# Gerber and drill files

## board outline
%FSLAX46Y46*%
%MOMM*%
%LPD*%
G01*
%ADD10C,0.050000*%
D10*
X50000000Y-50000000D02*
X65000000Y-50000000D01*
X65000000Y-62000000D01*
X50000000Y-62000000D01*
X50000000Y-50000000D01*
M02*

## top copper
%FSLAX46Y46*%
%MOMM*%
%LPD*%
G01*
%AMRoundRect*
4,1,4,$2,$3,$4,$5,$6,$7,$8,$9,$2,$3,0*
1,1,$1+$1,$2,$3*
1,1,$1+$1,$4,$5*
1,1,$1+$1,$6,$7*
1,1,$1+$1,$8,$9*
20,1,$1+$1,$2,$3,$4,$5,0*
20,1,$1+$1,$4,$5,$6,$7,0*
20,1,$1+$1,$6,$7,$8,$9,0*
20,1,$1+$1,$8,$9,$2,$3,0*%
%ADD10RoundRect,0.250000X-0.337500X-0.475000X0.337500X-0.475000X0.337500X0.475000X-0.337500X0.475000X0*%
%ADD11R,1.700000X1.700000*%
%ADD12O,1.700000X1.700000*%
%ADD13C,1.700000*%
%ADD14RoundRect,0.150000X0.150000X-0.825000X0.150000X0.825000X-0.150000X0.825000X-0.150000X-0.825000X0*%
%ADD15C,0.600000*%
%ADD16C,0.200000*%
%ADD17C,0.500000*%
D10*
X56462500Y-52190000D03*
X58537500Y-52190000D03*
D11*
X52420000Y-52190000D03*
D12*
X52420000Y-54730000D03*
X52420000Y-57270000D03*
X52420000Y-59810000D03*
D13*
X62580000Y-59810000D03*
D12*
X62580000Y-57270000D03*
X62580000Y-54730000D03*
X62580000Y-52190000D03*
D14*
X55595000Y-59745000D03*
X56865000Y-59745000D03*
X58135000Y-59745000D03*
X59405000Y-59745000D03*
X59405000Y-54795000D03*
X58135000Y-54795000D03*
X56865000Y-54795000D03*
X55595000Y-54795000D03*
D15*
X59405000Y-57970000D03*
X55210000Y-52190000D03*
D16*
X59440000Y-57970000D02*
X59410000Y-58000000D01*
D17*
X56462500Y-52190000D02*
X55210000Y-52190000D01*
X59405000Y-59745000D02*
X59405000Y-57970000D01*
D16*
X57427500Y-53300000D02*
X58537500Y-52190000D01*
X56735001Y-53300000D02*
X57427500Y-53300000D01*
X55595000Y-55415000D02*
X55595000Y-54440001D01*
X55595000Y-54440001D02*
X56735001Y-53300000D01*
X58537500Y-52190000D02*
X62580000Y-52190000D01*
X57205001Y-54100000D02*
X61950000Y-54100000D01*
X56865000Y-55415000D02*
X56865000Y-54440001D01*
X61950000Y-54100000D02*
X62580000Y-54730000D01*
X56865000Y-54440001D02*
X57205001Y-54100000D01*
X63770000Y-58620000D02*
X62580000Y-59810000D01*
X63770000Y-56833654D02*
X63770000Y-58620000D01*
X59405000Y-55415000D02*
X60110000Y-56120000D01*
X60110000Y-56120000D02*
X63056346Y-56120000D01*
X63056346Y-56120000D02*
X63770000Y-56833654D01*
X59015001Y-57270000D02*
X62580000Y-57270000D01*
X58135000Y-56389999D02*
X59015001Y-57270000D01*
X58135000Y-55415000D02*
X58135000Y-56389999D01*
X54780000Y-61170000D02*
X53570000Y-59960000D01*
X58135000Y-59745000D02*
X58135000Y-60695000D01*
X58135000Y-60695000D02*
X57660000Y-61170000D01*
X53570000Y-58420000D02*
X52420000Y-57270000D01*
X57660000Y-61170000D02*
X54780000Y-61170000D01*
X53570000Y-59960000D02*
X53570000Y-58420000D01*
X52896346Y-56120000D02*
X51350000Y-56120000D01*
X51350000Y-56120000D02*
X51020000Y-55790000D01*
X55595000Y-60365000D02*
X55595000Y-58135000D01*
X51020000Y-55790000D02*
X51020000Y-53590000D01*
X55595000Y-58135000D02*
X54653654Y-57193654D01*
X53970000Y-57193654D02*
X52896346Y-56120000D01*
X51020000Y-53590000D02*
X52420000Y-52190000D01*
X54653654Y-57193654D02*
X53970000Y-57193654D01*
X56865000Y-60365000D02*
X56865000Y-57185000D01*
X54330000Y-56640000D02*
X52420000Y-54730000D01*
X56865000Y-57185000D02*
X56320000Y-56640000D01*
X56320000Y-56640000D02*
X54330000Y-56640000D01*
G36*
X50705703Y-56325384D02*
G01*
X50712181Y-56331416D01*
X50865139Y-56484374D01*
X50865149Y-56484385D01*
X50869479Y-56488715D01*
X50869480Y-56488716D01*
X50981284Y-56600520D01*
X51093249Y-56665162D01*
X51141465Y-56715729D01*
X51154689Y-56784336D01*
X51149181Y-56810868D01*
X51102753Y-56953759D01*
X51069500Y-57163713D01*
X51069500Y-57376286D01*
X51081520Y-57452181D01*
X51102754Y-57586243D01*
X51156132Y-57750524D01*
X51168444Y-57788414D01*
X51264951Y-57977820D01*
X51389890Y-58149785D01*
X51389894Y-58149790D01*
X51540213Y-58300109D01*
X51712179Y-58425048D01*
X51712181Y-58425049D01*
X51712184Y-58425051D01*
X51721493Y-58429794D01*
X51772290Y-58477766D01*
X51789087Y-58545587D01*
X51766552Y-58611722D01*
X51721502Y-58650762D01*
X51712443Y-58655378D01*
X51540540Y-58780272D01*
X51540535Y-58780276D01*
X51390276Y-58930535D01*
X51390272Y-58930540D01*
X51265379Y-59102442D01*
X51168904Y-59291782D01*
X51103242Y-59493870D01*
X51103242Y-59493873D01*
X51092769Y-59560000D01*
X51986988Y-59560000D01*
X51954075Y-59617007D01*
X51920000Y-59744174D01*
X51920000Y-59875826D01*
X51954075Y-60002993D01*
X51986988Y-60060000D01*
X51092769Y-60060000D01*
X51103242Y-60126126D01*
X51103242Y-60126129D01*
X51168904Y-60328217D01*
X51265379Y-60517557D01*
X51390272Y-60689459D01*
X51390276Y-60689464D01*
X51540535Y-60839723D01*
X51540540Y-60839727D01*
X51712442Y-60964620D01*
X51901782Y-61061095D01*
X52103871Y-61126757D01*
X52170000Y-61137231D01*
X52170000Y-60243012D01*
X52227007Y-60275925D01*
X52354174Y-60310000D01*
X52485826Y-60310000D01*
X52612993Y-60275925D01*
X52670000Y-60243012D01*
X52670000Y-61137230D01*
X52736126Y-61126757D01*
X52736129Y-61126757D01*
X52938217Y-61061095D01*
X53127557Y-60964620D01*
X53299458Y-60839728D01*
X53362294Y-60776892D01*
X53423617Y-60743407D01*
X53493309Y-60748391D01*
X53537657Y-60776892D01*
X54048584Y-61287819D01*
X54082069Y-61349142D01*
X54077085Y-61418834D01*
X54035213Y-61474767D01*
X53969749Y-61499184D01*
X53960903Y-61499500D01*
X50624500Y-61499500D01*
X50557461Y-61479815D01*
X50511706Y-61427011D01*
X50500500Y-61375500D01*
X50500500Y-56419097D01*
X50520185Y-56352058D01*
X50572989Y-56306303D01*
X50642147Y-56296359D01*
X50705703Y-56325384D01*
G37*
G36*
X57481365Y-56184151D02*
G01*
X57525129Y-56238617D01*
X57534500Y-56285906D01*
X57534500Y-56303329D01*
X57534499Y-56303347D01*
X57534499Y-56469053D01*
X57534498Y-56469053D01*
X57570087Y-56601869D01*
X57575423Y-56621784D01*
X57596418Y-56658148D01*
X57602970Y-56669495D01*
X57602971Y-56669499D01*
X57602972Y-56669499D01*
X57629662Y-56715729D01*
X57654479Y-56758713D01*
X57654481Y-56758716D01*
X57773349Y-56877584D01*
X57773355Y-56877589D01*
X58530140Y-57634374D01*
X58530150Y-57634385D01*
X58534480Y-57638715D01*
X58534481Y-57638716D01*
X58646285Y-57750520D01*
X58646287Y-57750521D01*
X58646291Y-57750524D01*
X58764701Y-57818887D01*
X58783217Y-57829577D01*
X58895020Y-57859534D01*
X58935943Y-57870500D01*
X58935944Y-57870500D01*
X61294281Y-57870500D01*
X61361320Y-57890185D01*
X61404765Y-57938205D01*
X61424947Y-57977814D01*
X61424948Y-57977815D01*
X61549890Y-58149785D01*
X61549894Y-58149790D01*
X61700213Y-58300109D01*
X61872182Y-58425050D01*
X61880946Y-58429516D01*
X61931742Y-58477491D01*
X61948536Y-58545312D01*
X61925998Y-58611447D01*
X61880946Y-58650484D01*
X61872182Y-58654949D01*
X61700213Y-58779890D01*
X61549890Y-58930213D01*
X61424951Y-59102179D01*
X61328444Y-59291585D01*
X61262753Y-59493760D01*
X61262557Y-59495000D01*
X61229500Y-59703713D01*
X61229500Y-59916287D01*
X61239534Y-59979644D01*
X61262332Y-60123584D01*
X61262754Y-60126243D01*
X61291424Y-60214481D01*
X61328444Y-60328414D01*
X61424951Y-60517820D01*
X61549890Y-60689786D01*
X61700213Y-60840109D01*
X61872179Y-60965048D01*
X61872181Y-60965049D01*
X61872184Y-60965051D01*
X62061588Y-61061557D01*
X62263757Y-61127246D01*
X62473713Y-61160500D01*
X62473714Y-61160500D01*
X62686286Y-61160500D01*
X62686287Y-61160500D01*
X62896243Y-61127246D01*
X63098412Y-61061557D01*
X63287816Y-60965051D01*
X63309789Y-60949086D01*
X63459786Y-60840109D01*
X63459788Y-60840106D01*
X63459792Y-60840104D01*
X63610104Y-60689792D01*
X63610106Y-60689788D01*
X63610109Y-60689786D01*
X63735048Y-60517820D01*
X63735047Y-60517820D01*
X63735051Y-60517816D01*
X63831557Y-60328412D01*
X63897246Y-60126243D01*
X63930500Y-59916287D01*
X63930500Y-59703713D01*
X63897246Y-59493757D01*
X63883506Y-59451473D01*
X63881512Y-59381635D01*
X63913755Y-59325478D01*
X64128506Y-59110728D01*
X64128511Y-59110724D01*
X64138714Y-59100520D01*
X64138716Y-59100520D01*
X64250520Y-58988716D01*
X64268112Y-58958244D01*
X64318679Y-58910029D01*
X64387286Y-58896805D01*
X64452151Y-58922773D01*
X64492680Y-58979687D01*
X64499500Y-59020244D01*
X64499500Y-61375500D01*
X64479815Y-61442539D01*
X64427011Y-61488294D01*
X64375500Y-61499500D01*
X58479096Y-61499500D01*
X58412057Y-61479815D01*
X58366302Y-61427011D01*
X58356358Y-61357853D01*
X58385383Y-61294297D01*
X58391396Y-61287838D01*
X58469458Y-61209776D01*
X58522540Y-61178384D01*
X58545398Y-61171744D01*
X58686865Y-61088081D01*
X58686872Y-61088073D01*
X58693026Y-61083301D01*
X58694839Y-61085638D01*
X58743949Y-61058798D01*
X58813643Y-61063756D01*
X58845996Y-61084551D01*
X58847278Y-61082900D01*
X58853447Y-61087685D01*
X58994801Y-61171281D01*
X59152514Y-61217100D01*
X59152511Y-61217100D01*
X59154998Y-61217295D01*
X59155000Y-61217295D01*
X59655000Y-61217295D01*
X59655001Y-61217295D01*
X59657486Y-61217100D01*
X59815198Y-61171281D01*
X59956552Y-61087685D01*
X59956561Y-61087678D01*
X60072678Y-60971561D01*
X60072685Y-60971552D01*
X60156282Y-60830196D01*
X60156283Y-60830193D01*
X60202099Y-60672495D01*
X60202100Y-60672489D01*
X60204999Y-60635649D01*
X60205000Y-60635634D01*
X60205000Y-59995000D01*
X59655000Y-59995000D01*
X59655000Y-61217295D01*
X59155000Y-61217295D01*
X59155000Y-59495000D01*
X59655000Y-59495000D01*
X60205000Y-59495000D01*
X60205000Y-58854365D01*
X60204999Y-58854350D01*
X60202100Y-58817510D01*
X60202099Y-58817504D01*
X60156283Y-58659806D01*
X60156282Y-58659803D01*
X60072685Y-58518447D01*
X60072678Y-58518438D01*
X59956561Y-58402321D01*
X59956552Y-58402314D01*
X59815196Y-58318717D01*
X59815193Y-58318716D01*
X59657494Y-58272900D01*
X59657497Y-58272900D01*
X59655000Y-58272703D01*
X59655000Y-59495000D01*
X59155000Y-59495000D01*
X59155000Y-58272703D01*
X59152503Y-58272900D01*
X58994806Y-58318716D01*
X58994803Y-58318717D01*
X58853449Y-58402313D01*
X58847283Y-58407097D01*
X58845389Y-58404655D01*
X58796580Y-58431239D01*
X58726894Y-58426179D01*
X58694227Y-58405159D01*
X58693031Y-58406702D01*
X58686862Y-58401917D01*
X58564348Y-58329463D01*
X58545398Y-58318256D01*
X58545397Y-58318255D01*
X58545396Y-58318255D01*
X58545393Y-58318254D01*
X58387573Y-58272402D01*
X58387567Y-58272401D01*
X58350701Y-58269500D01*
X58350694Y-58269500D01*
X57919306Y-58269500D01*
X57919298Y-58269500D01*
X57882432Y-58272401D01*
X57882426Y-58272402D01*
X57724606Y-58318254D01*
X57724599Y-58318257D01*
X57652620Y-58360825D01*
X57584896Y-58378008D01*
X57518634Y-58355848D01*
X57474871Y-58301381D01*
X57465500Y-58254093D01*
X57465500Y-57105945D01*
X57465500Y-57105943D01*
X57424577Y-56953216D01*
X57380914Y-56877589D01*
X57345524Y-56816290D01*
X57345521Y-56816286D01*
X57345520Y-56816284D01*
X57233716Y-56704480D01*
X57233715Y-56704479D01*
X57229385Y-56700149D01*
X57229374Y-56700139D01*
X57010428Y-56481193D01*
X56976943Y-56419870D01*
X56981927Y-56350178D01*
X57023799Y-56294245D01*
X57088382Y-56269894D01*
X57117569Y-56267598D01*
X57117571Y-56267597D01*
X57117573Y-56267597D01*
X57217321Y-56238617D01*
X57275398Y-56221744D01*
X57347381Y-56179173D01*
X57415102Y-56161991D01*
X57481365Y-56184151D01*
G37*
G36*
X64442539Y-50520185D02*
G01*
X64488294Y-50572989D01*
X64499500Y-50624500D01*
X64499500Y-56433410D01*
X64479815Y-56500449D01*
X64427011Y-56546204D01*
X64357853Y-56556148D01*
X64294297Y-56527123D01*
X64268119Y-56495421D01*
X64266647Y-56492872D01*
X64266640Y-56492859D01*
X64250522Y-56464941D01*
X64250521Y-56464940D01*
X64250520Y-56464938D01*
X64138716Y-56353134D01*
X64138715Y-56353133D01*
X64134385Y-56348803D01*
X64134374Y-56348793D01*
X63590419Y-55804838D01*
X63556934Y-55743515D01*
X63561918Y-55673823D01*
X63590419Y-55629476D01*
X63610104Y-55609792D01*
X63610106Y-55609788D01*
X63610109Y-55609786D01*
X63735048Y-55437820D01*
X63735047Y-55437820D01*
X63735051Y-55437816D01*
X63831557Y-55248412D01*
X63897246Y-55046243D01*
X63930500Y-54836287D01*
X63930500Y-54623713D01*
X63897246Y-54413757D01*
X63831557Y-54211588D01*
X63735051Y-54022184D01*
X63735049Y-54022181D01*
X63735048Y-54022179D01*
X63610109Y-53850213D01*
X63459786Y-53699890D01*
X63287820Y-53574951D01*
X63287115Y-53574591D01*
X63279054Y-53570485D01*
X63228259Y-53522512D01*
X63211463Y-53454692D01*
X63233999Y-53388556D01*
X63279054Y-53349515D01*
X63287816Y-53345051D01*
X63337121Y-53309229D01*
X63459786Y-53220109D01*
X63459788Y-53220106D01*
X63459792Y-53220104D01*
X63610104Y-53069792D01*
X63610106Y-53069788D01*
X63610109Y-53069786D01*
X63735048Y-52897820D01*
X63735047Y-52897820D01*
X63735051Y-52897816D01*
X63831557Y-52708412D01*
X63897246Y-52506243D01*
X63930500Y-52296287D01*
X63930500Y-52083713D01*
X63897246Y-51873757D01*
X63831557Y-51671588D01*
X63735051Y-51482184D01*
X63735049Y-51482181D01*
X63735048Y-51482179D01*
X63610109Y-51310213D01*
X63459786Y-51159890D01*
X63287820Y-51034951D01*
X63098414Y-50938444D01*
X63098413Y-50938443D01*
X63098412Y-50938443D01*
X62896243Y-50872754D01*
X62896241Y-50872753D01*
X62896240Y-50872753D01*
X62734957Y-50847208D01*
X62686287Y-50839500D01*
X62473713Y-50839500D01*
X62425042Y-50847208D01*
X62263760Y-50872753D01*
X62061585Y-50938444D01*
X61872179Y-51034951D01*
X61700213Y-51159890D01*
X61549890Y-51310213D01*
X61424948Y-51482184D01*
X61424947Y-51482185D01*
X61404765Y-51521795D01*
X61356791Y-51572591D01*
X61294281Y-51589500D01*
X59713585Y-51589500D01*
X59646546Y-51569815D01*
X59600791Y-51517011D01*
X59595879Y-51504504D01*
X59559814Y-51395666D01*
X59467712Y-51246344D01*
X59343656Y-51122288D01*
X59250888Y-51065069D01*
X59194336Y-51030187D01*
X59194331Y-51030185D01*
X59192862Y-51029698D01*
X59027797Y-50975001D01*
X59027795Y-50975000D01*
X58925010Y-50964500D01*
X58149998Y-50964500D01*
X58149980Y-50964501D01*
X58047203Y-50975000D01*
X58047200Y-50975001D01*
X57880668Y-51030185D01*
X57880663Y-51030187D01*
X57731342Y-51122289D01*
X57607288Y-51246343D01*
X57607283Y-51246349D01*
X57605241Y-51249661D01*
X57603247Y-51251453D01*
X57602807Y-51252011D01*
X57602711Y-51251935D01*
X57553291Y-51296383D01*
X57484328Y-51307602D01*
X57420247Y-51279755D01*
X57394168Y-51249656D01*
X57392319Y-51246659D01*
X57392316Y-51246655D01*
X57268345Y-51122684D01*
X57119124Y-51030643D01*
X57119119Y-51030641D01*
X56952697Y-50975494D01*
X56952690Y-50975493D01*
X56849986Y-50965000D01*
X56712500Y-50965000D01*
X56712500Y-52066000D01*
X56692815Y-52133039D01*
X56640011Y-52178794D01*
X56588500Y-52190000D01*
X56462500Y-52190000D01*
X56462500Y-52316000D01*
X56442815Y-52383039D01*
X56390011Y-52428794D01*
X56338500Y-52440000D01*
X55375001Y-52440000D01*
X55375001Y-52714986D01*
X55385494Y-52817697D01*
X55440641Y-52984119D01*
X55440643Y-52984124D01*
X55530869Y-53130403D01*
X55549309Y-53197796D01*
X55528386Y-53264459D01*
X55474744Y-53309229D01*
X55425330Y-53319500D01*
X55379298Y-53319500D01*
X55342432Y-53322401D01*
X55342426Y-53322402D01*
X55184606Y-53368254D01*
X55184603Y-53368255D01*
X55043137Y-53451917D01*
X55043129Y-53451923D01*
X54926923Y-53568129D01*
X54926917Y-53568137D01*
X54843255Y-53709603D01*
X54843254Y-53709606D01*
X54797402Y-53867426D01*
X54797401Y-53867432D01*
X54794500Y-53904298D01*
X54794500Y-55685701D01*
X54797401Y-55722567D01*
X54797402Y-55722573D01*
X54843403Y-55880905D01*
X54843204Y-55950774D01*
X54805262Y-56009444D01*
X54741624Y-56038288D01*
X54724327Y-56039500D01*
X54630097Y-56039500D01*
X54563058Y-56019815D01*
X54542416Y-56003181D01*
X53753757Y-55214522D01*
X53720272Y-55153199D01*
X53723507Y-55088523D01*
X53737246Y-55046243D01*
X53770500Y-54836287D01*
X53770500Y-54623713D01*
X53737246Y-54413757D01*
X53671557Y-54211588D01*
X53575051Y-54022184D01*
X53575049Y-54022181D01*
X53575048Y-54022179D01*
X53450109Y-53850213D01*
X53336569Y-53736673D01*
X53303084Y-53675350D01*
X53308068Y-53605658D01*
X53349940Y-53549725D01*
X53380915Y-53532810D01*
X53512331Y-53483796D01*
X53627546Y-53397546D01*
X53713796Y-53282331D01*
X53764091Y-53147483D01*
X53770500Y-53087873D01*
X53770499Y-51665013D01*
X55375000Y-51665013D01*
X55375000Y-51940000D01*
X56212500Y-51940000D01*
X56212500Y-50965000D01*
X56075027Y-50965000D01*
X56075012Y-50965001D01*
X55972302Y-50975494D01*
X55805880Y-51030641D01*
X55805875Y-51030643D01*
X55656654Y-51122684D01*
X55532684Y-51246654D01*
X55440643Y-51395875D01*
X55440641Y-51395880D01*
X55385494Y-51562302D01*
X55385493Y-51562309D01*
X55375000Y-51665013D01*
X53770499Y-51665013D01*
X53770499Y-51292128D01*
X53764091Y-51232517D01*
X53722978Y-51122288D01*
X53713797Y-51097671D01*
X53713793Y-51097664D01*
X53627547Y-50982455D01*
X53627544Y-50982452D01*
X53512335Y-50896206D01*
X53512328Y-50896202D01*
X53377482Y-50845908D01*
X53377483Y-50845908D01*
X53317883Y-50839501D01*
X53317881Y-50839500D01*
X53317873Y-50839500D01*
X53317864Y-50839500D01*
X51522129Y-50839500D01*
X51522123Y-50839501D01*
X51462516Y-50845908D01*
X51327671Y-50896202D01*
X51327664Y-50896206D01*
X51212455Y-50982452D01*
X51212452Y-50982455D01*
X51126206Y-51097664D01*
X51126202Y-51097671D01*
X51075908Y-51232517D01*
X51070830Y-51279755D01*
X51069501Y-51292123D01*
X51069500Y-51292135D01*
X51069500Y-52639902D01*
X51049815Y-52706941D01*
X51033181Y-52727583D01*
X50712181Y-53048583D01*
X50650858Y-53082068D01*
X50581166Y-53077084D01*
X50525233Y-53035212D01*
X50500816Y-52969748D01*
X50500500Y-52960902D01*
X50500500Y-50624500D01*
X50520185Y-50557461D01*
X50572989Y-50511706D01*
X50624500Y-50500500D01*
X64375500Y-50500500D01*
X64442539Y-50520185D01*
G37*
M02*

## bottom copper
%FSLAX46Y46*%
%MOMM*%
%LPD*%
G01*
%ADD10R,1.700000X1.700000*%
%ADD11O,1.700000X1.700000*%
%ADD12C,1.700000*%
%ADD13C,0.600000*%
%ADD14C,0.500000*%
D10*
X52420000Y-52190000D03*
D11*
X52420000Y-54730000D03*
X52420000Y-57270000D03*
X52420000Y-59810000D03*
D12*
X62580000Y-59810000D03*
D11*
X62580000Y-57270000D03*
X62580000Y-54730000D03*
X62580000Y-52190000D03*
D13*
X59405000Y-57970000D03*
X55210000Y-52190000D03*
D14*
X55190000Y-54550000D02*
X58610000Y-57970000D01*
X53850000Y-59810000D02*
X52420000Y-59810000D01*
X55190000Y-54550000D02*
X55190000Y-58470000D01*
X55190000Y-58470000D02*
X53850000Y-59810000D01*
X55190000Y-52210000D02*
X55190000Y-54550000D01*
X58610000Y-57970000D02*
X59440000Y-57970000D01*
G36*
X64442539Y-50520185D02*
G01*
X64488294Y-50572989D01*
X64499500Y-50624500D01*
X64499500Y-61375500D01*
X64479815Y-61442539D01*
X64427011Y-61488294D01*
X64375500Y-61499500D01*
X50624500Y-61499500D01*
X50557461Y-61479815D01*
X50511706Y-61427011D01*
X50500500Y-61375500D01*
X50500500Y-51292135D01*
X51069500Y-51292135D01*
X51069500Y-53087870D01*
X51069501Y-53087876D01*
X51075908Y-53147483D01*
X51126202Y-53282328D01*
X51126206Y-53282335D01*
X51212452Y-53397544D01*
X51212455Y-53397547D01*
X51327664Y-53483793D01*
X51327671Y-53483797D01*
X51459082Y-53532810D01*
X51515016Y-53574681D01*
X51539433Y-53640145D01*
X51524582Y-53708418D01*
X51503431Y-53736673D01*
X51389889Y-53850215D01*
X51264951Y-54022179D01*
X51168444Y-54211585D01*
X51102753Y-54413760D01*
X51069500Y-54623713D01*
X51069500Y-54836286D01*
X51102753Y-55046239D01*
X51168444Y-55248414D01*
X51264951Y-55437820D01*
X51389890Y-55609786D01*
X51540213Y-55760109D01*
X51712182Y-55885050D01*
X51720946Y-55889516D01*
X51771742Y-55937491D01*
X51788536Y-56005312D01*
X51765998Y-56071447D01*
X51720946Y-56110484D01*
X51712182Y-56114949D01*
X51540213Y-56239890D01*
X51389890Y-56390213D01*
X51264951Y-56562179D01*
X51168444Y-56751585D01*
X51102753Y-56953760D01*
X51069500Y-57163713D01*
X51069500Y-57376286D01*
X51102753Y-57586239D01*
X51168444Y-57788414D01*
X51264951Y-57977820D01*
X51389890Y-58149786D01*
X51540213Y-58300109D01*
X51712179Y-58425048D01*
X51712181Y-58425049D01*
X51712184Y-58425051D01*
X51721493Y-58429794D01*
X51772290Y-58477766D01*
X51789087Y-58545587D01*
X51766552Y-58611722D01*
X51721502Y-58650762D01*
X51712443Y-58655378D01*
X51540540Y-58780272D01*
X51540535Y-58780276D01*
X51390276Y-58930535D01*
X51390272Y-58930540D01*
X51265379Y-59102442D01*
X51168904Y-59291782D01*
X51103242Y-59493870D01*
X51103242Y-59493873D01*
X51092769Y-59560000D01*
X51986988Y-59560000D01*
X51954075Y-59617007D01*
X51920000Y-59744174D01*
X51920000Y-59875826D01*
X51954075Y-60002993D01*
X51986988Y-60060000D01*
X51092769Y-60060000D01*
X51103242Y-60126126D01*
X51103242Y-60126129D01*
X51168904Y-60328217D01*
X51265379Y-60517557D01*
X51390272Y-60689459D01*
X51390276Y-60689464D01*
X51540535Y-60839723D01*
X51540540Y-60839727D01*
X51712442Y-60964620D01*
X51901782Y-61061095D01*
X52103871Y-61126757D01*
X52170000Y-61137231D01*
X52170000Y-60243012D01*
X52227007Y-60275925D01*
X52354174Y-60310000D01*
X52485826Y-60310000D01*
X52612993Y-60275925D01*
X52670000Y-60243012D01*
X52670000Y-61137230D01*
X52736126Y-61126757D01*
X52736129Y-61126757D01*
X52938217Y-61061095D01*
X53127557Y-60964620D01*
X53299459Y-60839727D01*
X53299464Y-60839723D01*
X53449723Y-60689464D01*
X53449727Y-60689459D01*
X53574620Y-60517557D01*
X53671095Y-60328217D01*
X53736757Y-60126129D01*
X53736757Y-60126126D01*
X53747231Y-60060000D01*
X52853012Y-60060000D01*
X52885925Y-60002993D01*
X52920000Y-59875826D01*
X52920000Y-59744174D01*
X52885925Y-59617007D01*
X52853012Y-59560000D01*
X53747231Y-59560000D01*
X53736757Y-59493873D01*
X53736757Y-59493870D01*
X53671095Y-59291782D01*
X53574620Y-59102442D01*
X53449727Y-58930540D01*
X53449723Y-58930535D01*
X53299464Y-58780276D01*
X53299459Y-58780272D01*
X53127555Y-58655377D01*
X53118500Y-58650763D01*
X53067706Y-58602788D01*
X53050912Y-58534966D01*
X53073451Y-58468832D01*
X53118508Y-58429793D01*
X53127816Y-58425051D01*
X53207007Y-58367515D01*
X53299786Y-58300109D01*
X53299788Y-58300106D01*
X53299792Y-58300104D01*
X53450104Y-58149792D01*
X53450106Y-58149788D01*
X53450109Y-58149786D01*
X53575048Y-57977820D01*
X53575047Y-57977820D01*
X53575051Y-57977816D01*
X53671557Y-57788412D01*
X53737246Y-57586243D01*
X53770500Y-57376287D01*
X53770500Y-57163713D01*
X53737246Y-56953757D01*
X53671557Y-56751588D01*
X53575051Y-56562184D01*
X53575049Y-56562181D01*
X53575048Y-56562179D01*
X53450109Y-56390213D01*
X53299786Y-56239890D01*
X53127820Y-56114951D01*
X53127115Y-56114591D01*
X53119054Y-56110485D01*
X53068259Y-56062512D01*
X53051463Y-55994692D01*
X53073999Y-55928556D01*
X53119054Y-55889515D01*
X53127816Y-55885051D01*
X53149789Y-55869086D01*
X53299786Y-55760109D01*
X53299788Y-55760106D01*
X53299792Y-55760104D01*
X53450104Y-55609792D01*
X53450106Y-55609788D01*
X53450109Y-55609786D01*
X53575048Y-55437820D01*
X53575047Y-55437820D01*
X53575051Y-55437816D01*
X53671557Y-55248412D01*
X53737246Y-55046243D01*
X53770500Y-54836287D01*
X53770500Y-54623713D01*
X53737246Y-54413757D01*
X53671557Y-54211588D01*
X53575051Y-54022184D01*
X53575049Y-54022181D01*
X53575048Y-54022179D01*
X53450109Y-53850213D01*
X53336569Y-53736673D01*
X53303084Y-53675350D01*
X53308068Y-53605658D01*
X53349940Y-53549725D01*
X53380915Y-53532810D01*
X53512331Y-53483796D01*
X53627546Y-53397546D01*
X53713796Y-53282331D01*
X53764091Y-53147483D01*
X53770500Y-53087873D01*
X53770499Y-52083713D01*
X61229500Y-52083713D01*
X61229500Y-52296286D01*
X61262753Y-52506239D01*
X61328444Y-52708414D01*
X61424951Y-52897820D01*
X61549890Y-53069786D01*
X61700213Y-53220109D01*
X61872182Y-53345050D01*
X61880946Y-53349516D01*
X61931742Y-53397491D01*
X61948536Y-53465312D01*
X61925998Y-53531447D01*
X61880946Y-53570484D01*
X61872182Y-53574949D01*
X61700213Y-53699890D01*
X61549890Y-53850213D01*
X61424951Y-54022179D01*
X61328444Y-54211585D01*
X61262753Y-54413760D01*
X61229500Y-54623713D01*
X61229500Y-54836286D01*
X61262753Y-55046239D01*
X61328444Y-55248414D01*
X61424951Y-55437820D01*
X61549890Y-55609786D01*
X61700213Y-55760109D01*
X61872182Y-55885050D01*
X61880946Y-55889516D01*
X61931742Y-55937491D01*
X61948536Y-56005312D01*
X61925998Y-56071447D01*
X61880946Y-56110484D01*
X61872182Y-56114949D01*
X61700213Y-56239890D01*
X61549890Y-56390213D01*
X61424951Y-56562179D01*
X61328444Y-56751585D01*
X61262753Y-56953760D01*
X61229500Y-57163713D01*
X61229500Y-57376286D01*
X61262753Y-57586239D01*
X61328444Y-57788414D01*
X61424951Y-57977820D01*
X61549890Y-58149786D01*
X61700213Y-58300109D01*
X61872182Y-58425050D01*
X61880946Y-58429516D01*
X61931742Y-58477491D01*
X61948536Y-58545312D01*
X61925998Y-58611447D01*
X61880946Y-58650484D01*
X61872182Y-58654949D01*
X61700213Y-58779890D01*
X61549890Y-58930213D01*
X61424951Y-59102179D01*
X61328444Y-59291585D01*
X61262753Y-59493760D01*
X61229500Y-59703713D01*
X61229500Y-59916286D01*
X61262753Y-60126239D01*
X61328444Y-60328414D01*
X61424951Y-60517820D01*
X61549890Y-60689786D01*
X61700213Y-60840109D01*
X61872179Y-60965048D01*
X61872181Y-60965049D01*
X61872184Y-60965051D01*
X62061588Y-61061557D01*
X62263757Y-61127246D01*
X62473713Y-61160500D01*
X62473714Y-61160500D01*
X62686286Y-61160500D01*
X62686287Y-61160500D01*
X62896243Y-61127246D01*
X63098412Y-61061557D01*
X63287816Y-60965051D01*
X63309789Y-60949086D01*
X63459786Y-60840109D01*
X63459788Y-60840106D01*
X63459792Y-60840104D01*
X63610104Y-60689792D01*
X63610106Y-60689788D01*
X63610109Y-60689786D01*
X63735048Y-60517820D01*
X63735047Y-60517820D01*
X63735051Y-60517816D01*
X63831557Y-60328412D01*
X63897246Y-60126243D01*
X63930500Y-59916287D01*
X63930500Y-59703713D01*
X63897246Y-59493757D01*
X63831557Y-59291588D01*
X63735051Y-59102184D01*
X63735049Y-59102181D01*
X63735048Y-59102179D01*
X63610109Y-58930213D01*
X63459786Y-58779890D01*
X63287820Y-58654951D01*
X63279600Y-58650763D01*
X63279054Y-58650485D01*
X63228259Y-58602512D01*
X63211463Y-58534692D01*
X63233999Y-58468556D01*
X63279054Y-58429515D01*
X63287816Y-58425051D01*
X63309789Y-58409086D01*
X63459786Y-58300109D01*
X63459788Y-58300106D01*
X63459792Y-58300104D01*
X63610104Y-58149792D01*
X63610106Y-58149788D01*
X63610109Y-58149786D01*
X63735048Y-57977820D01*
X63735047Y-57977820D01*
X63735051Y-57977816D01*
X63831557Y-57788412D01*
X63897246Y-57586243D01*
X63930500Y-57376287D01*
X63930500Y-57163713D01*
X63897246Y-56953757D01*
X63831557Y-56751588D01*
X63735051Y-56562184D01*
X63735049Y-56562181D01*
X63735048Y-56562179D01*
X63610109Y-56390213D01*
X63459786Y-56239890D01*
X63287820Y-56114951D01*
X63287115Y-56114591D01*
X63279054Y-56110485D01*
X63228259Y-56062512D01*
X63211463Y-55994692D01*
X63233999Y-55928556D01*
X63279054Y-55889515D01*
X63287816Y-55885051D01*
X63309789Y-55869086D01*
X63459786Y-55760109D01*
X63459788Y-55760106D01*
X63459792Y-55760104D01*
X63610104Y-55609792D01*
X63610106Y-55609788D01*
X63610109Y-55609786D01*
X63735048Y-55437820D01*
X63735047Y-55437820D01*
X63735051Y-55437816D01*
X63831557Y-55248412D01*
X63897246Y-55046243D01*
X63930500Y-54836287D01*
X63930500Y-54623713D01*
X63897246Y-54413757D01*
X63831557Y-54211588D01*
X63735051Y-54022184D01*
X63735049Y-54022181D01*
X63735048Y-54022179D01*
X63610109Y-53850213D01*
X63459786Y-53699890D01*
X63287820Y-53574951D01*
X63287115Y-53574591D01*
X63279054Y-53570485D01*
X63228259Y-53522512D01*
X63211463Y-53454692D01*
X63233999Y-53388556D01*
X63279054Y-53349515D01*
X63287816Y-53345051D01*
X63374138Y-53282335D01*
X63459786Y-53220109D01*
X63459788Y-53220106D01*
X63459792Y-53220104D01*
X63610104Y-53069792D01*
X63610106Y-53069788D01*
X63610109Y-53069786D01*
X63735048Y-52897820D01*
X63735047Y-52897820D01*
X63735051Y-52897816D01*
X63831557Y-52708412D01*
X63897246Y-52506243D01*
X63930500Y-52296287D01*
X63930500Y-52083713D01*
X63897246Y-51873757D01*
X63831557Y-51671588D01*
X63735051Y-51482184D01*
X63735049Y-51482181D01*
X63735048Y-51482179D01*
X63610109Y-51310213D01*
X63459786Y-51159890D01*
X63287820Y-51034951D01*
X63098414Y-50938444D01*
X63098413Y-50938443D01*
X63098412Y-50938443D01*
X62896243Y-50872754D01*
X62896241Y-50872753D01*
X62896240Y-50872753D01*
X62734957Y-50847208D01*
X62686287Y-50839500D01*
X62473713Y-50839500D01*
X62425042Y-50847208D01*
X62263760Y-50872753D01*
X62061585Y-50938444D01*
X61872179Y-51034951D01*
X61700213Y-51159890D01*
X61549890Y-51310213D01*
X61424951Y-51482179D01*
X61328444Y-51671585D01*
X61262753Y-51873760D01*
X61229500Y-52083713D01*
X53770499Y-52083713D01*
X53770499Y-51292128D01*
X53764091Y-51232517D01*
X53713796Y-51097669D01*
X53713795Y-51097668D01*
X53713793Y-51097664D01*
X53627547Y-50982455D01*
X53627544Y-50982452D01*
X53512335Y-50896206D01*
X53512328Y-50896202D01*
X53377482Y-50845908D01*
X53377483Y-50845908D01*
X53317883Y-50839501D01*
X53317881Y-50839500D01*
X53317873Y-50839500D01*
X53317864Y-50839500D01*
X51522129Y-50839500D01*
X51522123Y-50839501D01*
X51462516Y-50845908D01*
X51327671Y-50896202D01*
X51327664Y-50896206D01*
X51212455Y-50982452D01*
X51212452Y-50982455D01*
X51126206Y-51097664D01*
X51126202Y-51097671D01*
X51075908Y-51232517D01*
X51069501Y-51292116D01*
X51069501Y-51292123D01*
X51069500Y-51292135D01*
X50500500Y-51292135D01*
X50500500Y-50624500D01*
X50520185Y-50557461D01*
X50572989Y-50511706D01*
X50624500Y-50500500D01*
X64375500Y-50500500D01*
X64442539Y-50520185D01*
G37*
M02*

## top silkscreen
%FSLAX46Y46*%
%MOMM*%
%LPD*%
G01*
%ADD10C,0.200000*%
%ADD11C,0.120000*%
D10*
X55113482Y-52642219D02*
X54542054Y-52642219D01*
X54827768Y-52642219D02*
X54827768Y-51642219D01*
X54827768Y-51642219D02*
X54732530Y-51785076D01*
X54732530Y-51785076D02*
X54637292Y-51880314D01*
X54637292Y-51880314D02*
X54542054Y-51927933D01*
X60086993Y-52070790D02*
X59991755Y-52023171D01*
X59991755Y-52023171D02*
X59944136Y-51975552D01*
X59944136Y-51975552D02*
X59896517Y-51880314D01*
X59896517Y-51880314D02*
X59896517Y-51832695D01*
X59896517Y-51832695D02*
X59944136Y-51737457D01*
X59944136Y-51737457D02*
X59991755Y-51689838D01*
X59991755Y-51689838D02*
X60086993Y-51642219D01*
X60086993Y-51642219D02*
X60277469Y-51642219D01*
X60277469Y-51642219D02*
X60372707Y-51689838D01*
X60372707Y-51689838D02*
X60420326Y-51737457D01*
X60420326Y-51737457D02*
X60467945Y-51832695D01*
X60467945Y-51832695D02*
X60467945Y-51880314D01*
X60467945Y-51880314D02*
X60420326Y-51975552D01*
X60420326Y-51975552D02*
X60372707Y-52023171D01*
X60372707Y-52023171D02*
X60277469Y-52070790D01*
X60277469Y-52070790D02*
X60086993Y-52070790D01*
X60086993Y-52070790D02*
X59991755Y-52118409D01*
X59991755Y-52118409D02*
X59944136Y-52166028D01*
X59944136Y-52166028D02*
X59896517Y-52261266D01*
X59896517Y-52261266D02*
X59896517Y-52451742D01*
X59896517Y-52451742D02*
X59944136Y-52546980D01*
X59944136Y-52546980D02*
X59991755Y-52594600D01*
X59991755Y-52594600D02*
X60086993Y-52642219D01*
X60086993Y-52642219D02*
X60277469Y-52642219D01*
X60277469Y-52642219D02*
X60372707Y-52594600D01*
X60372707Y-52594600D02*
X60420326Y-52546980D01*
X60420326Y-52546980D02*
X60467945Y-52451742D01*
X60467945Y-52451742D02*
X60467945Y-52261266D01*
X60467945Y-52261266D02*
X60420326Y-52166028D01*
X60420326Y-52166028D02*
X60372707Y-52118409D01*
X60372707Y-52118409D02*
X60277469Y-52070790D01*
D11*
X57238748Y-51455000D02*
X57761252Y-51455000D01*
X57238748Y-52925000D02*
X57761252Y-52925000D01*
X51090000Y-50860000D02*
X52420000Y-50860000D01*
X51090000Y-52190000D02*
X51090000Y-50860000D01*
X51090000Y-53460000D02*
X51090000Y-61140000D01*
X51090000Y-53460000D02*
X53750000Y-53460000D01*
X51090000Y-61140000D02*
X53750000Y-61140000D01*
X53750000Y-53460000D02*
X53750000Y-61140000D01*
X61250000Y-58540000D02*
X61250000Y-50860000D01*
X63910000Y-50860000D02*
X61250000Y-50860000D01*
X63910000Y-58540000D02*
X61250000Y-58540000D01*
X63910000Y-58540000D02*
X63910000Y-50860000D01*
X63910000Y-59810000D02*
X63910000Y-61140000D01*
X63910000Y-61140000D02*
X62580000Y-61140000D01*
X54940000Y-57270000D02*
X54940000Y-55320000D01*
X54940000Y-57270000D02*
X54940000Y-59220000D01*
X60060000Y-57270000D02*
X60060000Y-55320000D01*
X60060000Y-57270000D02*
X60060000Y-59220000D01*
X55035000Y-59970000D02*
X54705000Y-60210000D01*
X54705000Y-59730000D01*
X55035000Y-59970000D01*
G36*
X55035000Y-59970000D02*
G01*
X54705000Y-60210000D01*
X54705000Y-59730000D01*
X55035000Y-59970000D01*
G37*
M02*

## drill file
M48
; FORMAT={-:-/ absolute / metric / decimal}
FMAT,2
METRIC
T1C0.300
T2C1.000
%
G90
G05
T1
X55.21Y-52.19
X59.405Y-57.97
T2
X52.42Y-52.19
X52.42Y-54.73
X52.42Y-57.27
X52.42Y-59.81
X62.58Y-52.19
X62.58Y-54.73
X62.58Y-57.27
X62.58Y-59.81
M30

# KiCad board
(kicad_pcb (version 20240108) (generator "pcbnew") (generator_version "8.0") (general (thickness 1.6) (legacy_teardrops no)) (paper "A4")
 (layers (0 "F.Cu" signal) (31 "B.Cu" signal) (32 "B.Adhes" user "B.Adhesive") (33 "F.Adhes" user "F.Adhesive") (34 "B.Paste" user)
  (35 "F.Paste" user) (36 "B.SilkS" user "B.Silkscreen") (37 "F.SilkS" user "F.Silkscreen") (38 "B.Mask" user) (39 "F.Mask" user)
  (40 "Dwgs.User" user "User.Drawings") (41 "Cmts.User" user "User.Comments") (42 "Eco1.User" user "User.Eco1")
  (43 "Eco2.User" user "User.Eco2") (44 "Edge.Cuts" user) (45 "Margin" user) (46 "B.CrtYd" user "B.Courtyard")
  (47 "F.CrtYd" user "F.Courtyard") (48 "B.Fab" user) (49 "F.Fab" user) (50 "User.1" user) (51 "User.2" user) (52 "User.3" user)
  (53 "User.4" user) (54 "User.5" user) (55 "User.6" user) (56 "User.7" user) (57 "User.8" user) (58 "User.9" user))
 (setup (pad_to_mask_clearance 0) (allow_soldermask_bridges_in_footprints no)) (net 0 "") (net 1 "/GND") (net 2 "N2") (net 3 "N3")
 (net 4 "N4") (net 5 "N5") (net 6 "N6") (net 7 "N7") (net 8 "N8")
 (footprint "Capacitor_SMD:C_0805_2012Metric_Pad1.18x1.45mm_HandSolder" (layer "F.Cu") (at 57.5 52.19)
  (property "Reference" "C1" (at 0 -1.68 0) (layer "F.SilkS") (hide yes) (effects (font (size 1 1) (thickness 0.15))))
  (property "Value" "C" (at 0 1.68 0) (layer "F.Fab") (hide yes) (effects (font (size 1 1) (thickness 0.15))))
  (fp_line (start -0.261252 -0.735) (end 0.261252 -0.735) (stroke (width 0.12) (type solid)) (layer "F.SilkS"))
  (fp_line (start -0.261252 0.735) (end 0.261252 0.735) (stroke (width 0.12) (type solid)) (layer "F.SilkS"))
  (pad "1" smd roundrect (at -1.0375 0) (size 1.175 1.45) (layers "F.Cu" "F.Paste" "F.Mask") (roundrect_rratio 0.212766) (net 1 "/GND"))
  (pad "2" smd roundrect (at 1.0375 0) (size 1.175 1.45) (layers "F.Cu" "F.Paste" "F.Mask") (roundrect_rratio 0.212766) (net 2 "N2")))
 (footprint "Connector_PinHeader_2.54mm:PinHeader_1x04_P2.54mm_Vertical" (layer "F.Cu") (at 52.42 52.19)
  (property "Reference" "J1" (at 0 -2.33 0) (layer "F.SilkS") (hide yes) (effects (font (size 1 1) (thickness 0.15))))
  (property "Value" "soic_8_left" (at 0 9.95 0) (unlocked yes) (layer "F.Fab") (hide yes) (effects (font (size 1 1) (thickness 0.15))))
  (fp_line (start -1.33 -1.33) (end 0 -1.33) (stroke (width 0.12) (type solid)) (layer "F.SilkS"))
  (fp_line (start -1.33 0) (end -1.33 -1.33) (stroke (width 0.12) (type solid)) (layer "F.SilkS"))
  (fp_line (start -1.33 1.27) (end -1.33 8.95) (stroke (width 0.12) (type solid)) (layer "F.SilkS"))
  (fp_line (start -1.33 1.27) (end 1.33 1.27) (stroke (width 0.12) (type solid)) (layer "F.SilkS"))
  (fp_line (start -1.33 8.95) (end 1.33 8.95) (stroke (width 0.12) (type solid)) (layer "F.SilkS"))
  (fp_line (start 1.33 1.27) (end 1.33 8.95) (stroke (width 0.12) (type solid)) (layer "F.SilkS"))
  (pad "1" thru_hole rect (at 0 0) (size 1.7 1.7) (drill 1) (layers "*.Cu" "*.Mask") (remove_unused_layers no) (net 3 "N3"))
  (pad "2" thru_hole oval (at 0 2.54) (size 1.7 1.7) (drill 1) (layers "*.Cu" "*.Mask") (remove_unused_layers no) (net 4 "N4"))
  (pad "3" thru_hole oval (at 0 5.08) (size 1.7 1.7) (drill 1) (layers "*.Cu" "*.Mask") (remove_unused_layers no) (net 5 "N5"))
  (pad "4" thru_hole oval (at 0 7.62) (size 1.7 1.7) (drill 1) (layers "*.Cu" "*.Mask") (remove_unused_layers no) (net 1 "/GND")))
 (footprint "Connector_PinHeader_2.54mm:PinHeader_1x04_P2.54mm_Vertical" (layer "F.Cu") (at 62.58 59.81 180)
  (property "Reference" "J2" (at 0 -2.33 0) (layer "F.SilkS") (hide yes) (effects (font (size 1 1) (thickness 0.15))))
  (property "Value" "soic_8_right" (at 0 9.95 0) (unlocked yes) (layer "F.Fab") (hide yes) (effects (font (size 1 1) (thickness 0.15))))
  (fp_line (start 1.33 1.27) (end 1.33 8.95) (stroke (width 0.12) (type solid)) (layer "F.SilkS"))
  (fp_line (start -1.33 8.95) (end 1.33 8.95) (stroke (width 0.12) (type solid)) (layer "F.SilkS"))
  (fp_line (start -1.33 1.27) (end 1.33 1.27) (stroke (width 0.12) (type solid)) (layer "F.SilkS"))
  (fp_line (start -1.33 1.27) (end -1.33 8.95) (stroke (width 0.12) (type solid)) (layer "F.SilkS"))
  (fp_line (start -1.33 0) (end -1.33 -1.33) (stroke (width 0.12) (type solid)) (layer "F.SilkS"))
  (fp_line (start -1.33 -1.33) (end 0 -1.33) (stroke (width 0.12) (type solid)) (layer "F.SilkS"))
  (pad "1" thru_hole circle (at 0 0 180) (size 1.7 1.7) (drill 1) (layers "*.Cu" "*.Mask") (remove_unused_layers no) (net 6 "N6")
   (thermal_bridge_angle 90))
  (pad "2" thru_hole oval (at 0 2.54 180) (size 1.7 1.7) (drill 1) (layers "*.Cu" "*.Mask") (remove_unused_layers no) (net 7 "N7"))
  (pad "3" thru_hole oval (at 0 5.08 180) (size 1.7 1.7) (drill 1) (layers "*.Cu" "*.Mask") (remove_unused_layers no) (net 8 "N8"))
  (pad "4" thru_hole oval (at 0 7.62 180) (size 1.7 1.7) (drill 1) (layers "*.Cu" "*.Mask") (remove_unused_layers no) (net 2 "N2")))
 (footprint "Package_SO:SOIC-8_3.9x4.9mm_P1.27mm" (layer "F.Cu") (at 57.5 57.27 90)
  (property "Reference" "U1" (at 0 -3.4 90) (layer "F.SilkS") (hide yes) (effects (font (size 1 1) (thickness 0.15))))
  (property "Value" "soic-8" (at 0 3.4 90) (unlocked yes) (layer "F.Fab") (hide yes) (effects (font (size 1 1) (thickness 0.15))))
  (fp_line (start 0 -2.56) (end 1.95 -2.56) (stroke (width 0.12) (type solid)) (layer "F.SilkS"))
  (fp_line (start 0 -2.56) (end -1.95 -2.56) (stroke (width 0.12) (type solid)) (layer "F.SilkS"))
  (fp_line (start 0 2.56) (end 1.95 2.56) (stroke (width 0.12) (type solid)) (layer "F.SilkS"))
  (fp_line (start 0 2.56) (end -1.95 2.56) (stroke (width 0.12) (type solid)) (layer "F.SilkS"))
  (fp_poly
   (pts (xy -2.7 -2.465) (xy -2.94 -2.795) (xy -2.46 -2.795) (xy -2.7 -2.465)) (stroke (width 0.12) (type solid)) (fill solid)
   (layer "F.SilkS"))
  (pad "1" smd roundrect (at -2.475 -1.905 90) (size 1.95 0.6) (layers "F.Cu" "F.Paste" "F.Mask") (roundrect_rratio 0.25) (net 3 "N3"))
  (pad "2" smd roundrect (at -2.475 -0.635 90) (size 1.95 0.6) (layers "F.Cu" "F.Paste" "F.Mask") (roundrect_rratio 0.25) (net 4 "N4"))
  (pad "3" smd roundrect (at -2.475 0.635 90) (size 1.95 0.6) (layers "F.Cu" "F.Paste" "F.Mask") (roundrect_rratio 0.25) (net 5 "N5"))
  (pad "4" smd roundrect (at -2.475 1.905 90) (size 1.95 0.6) (layers "F.Cu" "F.Paste" "F.Mask") (roundrect_rratio 0.25) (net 1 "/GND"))
  (pad "5" smd roundrect (at 2.475 1.905 90) (size 1.95 0.6) (layers "F.Cu" "F.Paste" "F.Mask") (roundrect_rratio 0.25) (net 6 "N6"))
  (pad "6" smd roundrect (at 2.475 0.635 90) (size 1.95 0.6) (layers "F.Cu" "F.Paste" "F.Mask") (roundrect_rratio 0.25) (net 7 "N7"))
  (pad "7" smd roundrect (at 2.475 -0.635 90) (size 1.95 0.6) (layers "F.Cu" "F.Paste" "F.Mask") (roundrect_rratio 0.25) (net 8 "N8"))
  (pad "8" smd roundrect (at 2.475 -1.905 90) (size 1.95 0.6) (layers "F.Cu" "F.Paste" "F.Mask") (roundrect_rratio 0.25) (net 2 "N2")))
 (gr_rect (start 50 50) (end 65 62) (stroke (width 0.05) (type default)) (fill none) (layer "Edge.Cuts"))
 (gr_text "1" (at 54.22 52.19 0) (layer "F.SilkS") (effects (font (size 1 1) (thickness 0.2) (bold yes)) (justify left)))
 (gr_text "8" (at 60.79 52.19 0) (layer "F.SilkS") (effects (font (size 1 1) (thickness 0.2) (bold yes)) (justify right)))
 (segment (start 59.44 57.97) (end 59.41 58) (width 0.2) (layer "F.Cu") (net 1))
 (segment (start 56.4625 52.19) (end 55.21 52.19) (width 0.5) (layer "F.Cu") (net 1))
 (segment (start 59.405 59.745) (end 59.405 57.97) (width 0.5) (layer "F.Cu") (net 1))
 (via (at 59.405 57.97) (size 0.6) (drill 0.3) (layers "F.Cu" "B.Cu") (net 1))
 (via (at 55.21 52.19) (size 0.6) (drill 0.3) (layers "F.Cu" "B.Cu") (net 1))
 (segment (start 55.19 54.55) (end 58.61 57.97) (width 0.5) (layer "B.Cu") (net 1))
 (segment (start 53.85 59.81) (end 52.42 59.81) (width 0.5) (layer "B.Cu") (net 1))
 (segment (start 55.19 54.55) (end 55.19 58.47) (width 0.5) (layer "B.Cu") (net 1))
 (segment (start 55.19 58.47) (end 53.85 59.81) (width 0.5) (layer "B.Cu") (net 1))
 (segment (start 55.19 52.21) (end 55.19 54.55) (width 0.5) (layer "B.Cu") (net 1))
 (segment (start 58.61 57.97) (end 59.44 57.97) (width 0.5) (layer "B.Cu") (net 1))
 (segment (start 57.4275 53.3) (end 58.5375 52.19) (width 0.2) (layer "F.Cu") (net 2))
 (segment (start 56.735001 53.3) (end 57.4275 53.3) (width 0.2) (layer "F.Cu") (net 2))
 (segment (start 55.595 55.415) (end 55.595 54.440001) (width 0.2) (layer "F.Cu") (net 2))
 (segment (start 55.595 54.440001) (end 56.735001 53.3) (width 0.2) (layer "F.Cu") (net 2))
 (segment (start 58.5375 52.19) (end 62.58 52.19) (width 0.2) (layer "F.Cu") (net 2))
 (segment (start 57.205001 54.1) (end 61.95 54.1) (width 0.2) (layer "F.Cu") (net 8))
 (segment (start 56.865 55.415) (end 56.865 54.440001) (width 0.2) (layer "F.Cu") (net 8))
 (segment (start 61.95 54.1) (end 62.58 54.73) (width 0.2) (layer "F.Cu") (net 8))
 (segment (start 56.865 54.440001) (end 57.205001 54.1) (width 0.2) (layer "F.Cu") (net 8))
 (segment (start 63.77 58.62) (end 62.58 59.81) (width 0.2) (layer "F.Cu") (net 6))
 (segment (start 63.77 56.833654) (end 63.77 58.62) (width 0.2) (layer "F.Cu") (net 6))
 (segment (start 59.405 55.415) (end 60.11 56.12) (width 0.2) (layer "F.Cu") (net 6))
 (segment (start 60.11 56.12) (end 63.056346 56.12) (width 0.2) (layer "F.Cu") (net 6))
 (segment (start 63.056346 56.12) (end 63.77 56.833654) (width 0.2) (layer "F.Cu") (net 6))
 (segment (start 59.015001 57.27) (end 62.58 57.27) (width 0.2) (layer "F.Cu") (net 7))
 (segment (start 58.135 56.389999) (end 59.015001 57.27) (width 0.2) (layer "F.Cu") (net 7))
 (segment (start 58.135 55.415) (end 58.135 56.389999) (width 0.2) (layer "F.Cu") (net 7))
 (segment (start 54.78 61.17) (end 53.57 59.96) (width 0.2) (layer "F.Cu") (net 5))
 (segment (start 58.135 59.745) (end 58.135 60.695) (width 0.2) (layer "F.Cu") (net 5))
 (segment (start 58.135 60.695) (end 57.66 61.17) (width 0.2) (layer "F.Cu") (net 5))
 (segment (start 53.57 58.42) (end 52.42 57.27) (width 0.2) (layer "F.Cu") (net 5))
 (segment (start 57.66 61.17) (end 54.78 61.17) (width 0.2) (layer "F.Cu") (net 5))
 (segment (start 53.57 59.96) (end 53.57 58.42) (width 0.2) (layer "F.Cu") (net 5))
 (segment (start 52.896346 56.12) (end 51.35 56.12) (width 0.2) (layer "F.Cu") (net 3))
 (segment (start 51.35 56.12) (end 51.02 55.79) (width 0.2) (layer "F.Cu") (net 3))
 (segment (start 55.595 60.365) (end 55.595 58.135) (width 0.2) (layer "F.Cu") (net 3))
 (segment (start 51.02 55.79) (end 51.02 53.59) (width 0.2) (layer "F.Cu") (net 3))
 (segment (start 55.595 58.135) (end 54.653654 57.193654) (width 0.2) (layer "F.Cu") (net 3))
 (segment (start 53.97 57.193654) (end 52.896346 56.12) (width 0.2) (layer "F.Cu") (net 3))
 (segment (start 51.02 53.59) (end 52.42 52.19) (width 0.2) (layer "F.Cu") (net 3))
 (segment (start 54.653654 57.193654) (end 53.97 57.193654) (width 0.2) (layer "F.Cu") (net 3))
 (segment (start 56.865 60.365) (end 56.865 57.185) (width 0.2) (layer "F.Cu") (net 4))
 (segment (start 54.33 56.64) (end 52.42 54.73) (width 0.2) (layer "F.Cu") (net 4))
 (segment (start 56.865 57.185) (end 56.32 56.64) (width 0.2) (layer "F.Cu") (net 4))
 (segment (start 56.32 56.64) (end 54.33 56.64) (width 0.2) (layer "F.Cu") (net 4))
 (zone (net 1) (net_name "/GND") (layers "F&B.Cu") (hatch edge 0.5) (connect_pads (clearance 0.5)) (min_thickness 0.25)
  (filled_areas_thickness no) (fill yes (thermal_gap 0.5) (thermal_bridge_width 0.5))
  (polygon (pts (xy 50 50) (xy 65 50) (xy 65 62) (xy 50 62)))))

